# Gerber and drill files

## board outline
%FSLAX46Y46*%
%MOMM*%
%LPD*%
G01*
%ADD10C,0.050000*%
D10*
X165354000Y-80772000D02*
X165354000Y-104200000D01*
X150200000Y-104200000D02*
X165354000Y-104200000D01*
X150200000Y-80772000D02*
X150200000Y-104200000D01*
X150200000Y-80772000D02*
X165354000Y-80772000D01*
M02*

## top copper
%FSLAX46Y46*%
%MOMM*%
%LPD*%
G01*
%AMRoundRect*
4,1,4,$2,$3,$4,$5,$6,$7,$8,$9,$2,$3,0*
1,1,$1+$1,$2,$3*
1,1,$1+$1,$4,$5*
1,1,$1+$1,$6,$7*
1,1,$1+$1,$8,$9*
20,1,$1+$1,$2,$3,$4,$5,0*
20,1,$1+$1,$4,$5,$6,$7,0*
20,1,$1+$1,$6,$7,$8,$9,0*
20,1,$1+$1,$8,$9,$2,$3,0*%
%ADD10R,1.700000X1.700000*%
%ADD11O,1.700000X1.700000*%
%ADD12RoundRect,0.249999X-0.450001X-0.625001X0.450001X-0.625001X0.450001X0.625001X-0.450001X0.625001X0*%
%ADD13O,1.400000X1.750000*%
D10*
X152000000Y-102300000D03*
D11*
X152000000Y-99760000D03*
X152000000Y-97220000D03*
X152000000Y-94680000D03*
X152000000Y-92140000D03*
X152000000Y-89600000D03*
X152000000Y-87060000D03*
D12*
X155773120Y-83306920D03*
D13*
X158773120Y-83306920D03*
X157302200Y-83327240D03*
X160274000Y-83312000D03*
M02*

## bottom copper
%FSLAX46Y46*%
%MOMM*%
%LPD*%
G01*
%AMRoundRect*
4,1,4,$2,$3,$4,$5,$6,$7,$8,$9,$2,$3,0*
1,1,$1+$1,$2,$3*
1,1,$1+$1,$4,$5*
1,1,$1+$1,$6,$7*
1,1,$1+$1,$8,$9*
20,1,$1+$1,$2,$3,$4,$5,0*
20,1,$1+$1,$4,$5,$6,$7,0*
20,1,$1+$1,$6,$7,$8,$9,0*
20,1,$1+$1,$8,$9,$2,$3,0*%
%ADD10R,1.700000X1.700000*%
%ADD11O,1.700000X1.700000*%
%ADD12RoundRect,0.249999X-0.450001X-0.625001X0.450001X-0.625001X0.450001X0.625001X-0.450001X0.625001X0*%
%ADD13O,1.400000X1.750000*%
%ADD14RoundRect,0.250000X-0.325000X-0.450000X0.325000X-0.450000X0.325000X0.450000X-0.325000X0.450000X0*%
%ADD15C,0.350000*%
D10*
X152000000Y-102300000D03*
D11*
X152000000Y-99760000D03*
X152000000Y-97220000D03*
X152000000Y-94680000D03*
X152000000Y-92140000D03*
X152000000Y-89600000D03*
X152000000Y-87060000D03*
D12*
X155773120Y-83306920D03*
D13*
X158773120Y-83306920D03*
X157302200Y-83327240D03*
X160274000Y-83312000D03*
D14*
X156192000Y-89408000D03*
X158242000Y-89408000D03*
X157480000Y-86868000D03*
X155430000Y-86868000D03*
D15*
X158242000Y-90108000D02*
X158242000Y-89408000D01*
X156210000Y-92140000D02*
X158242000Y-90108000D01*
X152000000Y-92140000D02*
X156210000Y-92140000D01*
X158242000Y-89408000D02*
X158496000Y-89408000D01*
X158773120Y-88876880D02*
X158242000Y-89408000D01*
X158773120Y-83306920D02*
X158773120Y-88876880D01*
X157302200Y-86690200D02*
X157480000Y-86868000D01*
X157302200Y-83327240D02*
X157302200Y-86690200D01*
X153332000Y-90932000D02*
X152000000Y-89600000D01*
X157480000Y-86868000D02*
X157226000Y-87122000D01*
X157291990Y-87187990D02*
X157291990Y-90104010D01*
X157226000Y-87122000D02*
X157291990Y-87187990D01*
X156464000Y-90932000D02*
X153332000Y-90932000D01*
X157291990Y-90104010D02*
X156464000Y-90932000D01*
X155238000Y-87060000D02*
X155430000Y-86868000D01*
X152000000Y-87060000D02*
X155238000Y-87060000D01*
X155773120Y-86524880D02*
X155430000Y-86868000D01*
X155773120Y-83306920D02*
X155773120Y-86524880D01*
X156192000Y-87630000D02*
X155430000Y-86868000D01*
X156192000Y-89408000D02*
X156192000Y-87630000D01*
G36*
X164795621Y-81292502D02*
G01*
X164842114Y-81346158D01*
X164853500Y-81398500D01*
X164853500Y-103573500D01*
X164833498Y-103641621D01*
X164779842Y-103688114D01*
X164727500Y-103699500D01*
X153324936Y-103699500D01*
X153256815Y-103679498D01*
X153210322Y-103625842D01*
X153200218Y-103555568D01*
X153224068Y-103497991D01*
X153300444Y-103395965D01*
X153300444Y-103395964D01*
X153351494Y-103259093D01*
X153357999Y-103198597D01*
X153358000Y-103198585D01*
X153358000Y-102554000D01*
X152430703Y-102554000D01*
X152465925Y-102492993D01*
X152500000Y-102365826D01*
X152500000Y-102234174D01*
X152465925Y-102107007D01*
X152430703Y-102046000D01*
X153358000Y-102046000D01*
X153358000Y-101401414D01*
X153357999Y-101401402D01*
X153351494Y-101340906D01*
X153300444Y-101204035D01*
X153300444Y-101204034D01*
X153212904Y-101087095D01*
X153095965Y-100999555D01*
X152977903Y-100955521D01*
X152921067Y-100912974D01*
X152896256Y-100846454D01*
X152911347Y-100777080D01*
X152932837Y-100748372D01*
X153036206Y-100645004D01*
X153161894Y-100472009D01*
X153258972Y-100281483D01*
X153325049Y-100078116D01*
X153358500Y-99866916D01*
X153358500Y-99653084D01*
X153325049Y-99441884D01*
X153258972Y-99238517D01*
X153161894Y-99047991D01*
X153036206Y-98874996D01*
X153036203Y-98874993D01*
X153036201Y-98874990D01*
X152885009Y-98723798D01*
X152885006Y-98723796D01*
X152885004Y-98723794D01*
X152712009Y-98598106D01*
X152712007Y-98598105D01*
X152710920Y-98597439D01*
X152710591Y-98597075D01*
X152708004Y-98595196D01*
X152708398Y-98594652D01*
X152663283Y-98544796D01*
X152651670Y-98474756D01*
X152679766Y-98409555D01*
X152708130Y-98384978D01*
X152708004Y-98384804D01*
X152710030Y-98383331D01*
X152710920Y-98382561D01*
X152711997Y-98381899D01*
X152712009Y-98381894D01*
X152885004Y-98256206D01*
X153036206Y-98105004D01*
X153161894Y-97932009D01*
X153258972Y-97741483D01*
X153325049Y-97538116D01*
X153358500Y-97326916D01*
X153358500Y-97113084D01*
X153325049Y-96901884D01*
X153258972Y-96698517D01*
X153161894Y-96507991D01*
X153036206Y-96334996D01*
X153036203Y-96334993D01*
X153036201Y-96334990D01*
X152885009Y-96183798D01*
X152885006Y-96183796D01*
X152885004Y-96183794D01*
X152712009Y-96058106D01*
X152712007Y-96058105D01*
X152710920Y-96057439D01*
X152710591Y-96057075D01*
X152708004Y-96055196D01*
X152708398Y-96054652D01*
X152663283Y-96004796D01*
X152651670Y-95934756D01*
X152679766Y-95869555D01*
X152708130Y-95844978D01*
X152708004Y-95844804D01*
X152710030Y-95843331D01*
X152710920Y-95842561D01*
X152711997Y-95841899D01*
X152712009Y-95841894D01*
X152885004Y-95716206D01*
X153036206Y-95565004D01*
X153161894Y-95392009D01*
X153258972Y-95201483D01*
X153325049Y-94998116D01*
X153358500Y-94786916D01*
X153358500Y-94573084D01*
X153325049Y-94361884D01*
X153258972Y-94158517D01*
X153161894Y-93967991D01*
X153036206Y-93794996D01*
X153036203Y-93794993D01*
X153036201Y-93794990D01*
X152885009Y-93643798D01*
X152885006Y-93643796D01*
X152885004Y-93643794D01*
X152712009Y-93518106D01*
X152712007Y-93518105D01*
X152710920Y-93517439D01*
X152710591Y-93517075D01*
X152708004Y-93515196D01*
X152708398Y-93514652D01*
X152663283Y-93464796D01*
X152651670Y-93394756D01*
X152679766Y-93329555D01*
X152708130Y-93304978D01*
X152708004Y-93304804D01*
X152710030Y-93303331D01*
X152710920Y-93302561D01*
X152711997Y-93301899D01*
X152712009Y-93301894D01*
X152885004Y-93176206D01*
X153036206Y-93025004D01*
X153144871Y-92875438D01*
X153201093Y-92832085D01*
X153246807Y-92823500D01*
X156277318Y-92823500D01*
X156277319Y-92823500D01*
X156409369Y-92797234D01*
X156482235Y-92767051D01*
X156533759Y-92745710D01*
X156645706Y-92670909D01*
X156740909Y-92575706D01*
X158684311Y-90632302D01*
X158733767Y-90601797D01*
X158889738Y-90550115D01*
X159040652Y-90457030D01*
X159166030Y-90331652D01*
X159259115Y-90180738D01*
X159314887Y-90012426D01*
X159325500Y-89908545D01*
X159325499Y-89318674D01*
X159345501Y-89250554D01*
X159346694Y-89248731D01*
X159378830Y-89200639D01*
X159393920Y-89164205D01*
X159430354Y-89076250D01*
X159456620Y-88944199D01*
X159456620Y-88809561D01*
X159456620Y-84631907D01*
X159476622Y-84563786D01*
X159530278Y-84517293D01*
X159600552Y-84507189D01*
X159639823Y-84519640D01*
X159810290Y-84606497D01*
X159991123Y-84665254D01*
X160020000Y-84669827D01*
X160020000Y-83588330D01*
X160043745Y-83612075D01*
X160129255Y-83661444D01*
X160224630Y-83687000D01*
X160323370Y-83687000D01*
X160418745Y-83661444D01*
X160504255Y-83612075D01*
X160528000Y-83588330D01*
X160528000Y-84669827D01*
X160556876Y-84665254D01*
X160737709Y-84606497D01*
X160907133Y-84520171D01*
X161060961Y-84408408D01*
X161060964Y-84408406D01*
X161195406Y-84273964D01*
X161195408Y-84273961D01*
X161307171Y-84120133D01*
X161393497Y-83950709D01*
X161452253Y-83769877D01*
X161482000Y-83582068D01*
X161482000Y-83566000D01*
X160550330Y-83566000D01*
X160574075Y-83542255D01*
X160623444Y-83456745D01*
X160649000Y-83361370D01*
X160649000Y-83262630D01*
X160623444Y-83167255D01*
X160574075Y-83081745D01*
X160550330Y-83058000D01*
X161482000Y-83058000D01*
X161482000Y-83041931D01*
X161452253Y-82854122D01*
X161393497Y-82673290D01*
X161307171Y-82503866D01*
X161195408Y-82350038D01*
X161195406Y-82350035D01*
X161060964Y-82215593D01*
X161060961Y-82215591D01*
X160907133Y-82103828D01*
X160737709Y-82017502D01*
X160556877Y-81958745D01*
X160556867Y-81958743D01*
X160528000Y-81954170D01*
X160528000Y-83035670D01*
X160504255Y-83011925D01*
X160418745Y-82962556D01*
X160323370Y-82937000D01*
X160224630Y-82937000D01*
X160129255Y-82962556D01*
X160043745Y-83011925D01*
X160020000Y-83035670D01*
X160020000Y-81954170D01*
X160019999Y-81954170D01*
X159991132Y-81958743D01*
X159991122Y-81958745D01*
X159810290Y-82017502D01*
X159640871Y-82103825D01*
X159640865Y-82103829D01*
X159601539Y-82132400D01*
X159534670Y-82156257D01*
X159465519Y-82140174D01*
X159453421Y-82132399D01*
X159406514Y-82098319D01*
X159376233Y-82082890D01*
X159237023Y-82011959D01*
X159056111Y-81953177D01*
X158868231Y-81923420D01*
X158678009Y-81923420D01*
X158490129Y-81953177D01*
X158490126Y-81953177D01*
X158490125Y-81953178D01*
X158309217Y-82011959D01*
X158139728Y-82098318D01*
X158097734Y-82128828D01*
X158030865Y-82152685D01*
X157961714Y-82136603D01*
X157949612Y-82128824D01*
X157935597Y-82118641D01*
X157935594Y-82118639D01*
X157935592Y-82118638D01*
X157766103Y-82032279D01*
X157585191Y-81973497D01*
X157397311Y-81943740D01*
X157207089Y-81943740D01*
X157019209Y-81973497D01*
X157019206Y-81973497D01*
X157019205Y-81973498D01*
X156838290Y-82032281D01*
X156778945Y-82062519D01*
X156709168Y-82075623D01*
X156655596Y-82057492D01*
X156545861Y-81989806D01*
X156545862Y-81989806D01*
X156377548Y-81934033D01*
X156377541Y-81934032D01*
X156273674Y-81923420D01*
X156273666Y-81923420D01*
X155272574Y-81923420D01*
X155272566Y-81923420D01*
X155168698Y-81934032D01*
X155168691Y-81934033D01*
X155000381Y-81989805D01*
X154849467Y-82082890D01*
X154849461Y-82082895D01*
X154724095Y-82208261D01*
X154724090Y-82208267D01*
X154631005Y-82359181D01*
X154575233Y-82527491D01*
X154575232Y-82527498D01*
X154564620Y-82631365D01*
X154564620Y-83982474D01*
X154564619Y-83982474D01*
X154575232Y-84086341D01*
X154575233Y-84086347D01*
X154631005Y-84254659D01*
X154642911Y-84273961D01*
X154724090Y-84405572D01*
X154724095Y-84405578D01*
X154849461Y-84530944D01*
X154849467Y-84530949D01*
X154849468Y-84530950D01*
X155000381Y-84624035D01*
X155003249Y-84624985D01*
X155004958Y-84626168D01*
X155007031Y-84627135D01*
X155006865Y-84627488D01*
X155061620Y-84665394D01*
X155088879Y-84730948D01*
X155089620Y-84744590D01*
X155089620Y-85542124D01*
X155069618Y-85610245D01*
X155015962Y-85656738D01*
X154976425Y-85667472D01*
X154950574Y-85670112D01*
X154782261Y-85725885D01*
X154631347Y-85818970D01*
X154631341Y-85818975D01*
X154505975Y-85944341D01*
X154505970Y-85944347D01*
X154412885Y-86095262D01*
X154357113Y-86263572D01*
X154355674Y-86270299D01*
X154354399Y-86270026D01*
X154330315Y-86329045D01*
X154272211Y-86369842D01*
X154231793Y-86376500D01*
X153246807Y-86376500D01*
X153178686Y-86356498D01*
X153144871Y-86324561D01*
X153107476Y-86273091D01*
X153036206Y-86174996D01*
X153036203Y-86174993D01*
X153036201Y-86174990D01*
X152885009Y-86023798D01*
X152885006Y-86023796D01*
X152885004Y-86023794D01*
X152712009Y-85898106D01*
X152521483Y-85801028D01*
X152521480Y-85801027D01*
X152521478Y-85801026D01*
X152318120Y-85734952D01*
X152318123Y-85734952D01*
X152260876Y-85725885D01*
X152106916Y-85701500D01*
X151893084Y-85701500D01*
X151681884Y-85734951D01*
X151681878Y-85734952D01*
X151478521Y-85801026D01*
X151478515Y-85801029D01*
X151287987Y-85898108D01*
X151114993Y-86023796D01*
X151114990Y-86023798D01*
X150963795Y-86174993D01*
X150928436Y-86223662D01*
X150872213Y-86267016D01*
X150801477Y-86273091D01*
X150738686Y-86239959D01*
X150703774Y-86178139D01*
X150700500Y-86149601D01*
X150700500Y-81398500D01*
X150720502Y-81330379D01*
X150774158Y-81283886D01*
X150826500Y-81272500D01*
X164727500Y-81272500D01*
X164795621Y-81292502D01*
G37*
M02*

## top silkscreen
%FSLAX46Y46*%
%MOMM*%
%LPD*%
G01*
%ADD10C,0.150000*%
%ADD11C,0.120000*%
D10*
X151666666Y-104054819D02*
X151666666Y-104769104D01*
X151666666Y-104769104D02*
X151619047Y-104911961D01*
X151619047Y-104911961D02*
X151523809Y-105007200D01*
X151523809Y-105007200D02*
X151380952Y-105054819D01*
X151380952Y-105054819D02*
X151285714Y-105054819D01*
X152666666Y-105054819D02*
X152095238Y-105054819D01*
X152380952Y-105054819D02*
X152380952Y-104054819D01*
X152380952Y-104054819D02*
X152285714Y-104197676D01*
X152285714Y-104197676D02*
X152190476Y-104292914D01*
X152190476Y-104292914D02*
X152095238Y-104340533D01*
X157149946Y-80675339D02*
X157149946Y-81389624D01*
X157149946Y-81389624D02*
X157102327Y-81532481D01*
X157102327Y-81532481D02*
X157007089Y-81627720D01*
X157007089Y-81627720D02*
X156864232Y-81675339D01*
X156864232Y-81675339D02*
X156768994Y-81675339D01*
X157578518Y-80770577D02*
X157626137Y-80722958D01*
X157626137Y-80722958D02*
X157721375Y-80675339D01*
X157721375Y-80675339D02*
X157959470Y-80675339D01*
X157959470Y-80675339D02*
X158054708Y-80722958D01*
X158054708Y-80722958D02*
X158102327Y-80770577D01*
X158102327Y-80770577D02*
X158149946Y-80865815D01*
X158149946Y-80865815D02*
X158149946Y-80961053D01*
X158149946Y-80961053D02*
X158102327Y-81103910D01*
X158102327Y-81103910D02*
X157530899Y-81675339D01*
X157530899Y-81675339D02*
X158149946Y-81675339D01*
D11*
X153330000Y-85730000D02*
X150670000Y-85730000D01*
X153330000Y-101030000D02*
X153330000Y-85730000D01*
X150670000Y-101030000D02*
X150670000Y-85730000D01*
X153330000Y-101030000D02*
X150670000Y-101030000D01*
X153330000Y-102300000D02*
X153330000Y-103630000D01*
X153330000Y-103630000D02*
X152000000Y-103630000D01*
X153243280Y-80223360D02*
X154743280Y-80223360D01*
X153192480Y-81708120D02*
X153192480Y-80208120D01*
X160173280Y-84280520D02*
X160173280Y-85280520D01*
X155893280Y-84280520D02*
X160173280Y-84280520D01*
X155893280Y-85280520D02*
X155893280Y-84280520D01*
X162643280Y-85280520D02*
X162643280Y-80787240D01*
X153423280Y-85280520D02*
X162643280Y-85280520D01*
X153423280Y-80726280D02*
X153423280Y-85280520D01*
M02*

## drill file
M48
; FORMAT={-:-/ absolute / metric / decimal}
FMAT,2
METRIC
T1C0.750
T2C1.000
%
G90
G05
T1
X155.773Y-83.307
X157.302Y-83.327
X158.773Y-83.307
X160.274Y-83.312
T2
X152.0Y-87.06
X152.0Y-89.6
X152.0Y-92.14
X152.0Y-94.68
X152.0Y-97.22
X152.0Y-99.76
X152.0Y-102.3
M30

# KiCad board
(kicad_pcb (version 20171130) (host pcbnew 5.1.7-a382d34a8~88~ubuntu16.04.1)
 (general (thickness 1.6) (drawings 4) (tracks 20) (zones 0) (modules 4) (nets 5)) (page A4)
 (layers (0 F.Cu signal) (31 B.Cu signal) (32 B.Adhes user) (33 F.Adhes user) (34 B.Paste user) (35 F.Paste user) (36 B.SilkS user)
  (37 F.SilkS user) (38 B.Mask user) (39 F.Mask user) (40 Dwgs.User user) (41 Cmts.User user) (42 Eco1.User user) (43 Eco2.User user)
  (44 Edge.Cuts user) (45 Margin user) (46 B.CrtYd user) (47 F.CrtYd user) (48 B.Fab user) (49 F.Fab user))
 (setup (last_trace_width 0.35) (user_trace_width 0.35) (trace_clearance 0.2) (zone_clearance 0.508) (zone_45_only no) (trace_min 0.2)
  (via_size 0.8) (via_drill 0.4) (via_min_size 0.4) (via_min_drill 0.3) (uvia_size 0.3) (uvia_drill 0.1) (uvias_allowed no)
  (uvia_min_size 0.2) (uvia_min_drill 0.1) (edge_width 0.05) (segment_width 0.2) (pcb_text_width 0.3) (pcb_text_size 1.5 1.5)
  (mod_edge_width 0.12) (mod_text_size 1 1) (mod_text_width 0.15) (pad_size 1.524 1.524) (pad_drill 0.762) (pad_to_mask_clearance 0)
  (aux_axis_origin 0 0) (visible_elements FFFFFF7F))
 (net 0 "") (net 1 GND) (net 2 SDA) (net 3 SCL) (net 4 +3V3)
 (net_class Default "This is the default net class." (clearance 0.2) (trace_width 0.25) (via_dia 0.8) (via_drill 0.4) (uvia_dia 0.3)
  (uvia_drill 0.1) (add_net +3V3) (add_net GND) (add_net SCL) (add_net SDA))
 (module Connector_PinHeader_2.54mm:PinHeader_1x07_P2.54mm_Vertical (layer F.Cu) (at 152 102.3 180)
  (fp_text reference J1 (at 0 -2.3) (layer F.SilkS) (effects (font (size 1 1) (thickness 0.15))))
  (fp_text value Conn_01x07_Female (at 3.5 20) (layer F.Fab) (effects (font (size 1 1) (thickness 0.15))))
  (fp_line (start -1.33 16.57) (end 1.33 16.57) (layer F.SilkS) (width 0.12))
  (fp_line (start -1.33 1.27) (end -1.33 16.57) (layer F.SilkS) (width 0.12))
  (fp_line (start 1.33 1.27) (end 1.33 16.57) (layer F.SilkS) (width 0.12))
  (fp_line (start -1.33 1.27) (end 1.33 1.27) (layer F.SilkS) (width 0.12))
  (fp_line (start -1.33 0) (end -1.33 -1.33) (layer F.SilkS) (width 0.12))
  (fp_line (start -1.33 -1.33) (end 0 -1.33) (layer F.SilkS) (width 0.12))
  (pad 1 thru_hole rect (at 0 0 180) (size 1.7 1.7) (drill 1) (layers *.Cu *.Mask) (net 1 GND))
  (pad 2 thru_hole oval (at 0 2.54 180) (size 1.7 1.7) (drill 1) (layers *.Cu *.Mask))
  (pad 3 thru_hole oval (at 0 5.08 180) (size 1.7 1.7) (drill 1) (layers *.Cu *.Mask))
  (pad 4 thru_hole oval (at 0 7.62 180) (size 1.7 1.7) (drill 1) (layers *.Cu *.Mask))
  (pad 5 thru_hole oval (at 0 10.16 180) (size 1.7 1.7) (drill 1) (layers *.Cu *.Mask) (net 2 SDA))
  (pad 6 thru_hole oval (at 0 12.7 180) (size 1.7 1.7) (drill 1) (layers *.Cu *.Mask) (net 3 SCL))
  (pad 7 thru_hole oval (at 0 15.24 180) (size 1.7 1.7) (drill 1) (layers *.Cu *.Mask) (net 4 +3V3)))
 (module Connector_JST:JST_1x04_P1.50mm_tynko (layer F.Cu) (at 155.78328 77.82052)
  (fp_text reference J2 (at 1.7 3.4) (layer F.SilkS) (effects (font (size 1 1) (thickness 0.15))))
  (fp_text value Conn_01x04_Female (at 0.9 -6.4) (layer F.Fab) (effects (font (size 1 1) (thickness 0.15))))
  (fp_line (start -2.54 2.40284) (end -1.04 2.40284) (layer F.SilkS) (width 0.12))
  (fp_line (start -2.5908 3.8876) (end -2.5908 2.3876) (layer F.SilkS) (width 0.12))
  (fp_line (start 4.39 6.46) (end 4.39 7.46) (layer F.SilkS) (width 0.12))
  (fp_line (start 0.11 6.46) (end 4.39 6.46) (layer F.SilkS) (width 0.12))
  (fp_line (start 0.11 7.46) (end 0.11 6.46) (layer F.SilkS) (width 0.12))
  (fp_line (start 6.86 7.46) (end 6.86 2.96672) (layer F.SilkS) (width 0.12))
  (fp_line (start -2.36 7.46) (end 6.86 7.46) (layer F.SilkS) (width 0.12))
  (fp_line (start -2.36 2.90576) (end -2.36 7.46) (layer F.SilkS) (width 0.12))
  (pad 1 thru_hole roundrect (at -0.01016 5.4864) (size 1.4 1.75) (drill 0.75) (layers *.Cu *.Mask) (roundrect_rratio 0.178571) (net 4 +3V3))
  (pad 3 thru_hole oval (at 2.98984 5.4864) (size 1.4 1.75) (drill 0.75) (layers *.Cu *.Mask) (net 2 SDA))
  (pad 2 thru_hole oval (at 1.51892 5.50672) (size 1.4 1.75) (drill 0.75) (layers *.Cu *.Mask) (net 3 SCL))
  (pad 4 thru_hole oval (at 4.49072 5.49148) (size 1.4 1.75) (drill 0.75) (layers *.Cu *.Mask) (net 1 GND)))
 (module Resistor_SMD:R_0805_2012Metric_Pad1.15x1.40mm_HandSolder (layer B.Cu) (at 157.217 89.408)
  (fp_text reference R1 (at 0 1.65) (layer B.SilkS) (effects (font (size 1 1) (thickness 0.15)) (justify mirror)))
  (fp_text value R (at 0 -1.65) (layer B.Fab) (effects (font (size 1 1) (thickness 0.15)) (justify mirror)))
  (pad 1 smd roundrect (at -1.025 0) (size 1.15 1.4) (layers B.Cu B.Paste B.Mask) (roundrect_rratio 0.217391) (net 4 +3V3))
  (pad 2 smd roundrect (at 1.025 0) (size 1.15 1.4) (layers B.Cu B.Paste B.Mask) (roundrect_rratio 0.217391) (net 2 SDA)))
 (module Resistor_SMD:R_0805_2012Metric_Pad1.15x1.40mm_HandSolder (layer B.Cu) (at 156.455 86.868)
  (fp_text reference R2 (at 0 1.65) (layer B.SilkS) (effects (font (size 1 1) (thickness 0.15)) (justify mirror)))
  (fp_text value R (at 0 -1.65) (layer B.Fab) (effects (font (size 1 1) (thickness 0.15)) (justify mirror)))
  (pad 2 smd roundrect (at 1.025 0) (size 1.15 1.4) (layers B.Cu B.Paste B.Mask) (roundrect_rratio 0.217391) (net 3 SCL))
  (pad 1 smd roundrect (at -1.025 0) (size 1.15 1.4) (layers B.Cu B.Paste B.Mask) (roundrect_rratio 0.217391) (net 4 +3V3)))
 (gr_line (start 165.354 80.772) (end 165.354 104.2) (layer Edge.Cuts) (width 0.05))
 (gr_line (start 150.2 104.2) (end 165.354 104.2) (layer Edge.Cuts) (width 0.05))
 (gr_line (start 150.2 80.772) (end 150.2 104.2) (layer Edge.Cuts) (width 0.05))
 (gr_line (start 150.2 80.772) (end 165.354 80.772) (layer Edge.Cuts) (width 0.05))
 (segment (start 158.242 90.108) (end 158.242 89.408) (width 0.35) (layer B.Cu) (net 2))
 (segment (start 156.21 92.14) (end 158.242 90.108) (width 0.35) (layer B.Cu) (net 2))
 (segment (start 152 92.14) (end 156.21 92.14) (width 0.35) (layer B.Cu) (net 2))
 (segment (start 158.242 89.408) (end 158.496 89.408) (width 0.35) (layer B.Cu) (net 2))
 (segment (start 158.77312 88.87688) (end 158.242 89.408) (width 0.35) (layer B.Cu) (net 2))
 (segment (start 158.77312 83.30692) (end 158.77312 88.87688) (width 0.35) (layer B.Cu) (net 2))
 (segment (start 157.3022 86.6902) (end 157.48 86.868) (width 0.35) (layer B.Cu) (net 3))
 (segment (start 157.3022 83.32724) (end 157.3022 86.6902) (width 0.35) (layer B.Cu) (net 3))
 (segment (start 153.332 90.932) (end 152 89.6) (width 0.35) (layer B.Cu) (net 3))
 (segment (start 157.48 86.868) (end 157.226 87.122) (width 0.35) (layer B.Cu) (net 3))
 (segment (start 157.29199 87.18799) (end 157.29199 90.10401) (width 0.35) (layer B.Cu) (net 3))
 (segment (start 157.226 87.122) (end 157.29199 87.18799) (width 0.35) (layer B.Cu) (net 3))
 (segment (start 156.464 90.932) (end 153.332 90.932) (width 0.35) (layer B.Cu) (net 3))
 (segment (start 157.29199 90.10401) (end 156.464 90.932) (width 0.35) (layer B.Cu) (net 3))
 (segment (start 155.238 87.06) (end 155.43 86.868) (width 0.35) (layer B.Cu) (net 4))
 (segment (start 152 87.06) (end 155.238 87.06) (width 0.35) (layer B.Cu) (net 4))
 (segment (start 155.77312 86.52488) (end 155.43 86.868) (width 0.35) (layer B.Cu) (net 4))
 (segment (start 155.77312 83.30692) (end 155.77312 86.52488) (width 0.35) (layer B.Cu) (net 4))
 (segment (start 156.192 87.63) (end 155.43 86.868) (width 0.35) (layer B.Cu) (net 4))
 (segment (start 156.192 89.408) (end 156.192 87.63) (width 0.35) (layer B.Cu) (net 4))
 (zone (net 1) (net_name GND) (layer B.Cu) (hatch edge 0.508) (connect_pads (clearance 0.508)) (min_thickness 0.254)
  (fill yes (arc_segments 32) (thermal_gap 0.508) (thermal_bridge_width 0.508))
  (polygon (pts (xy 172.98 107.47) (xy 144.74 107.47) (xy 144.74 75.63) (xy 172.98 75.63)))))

